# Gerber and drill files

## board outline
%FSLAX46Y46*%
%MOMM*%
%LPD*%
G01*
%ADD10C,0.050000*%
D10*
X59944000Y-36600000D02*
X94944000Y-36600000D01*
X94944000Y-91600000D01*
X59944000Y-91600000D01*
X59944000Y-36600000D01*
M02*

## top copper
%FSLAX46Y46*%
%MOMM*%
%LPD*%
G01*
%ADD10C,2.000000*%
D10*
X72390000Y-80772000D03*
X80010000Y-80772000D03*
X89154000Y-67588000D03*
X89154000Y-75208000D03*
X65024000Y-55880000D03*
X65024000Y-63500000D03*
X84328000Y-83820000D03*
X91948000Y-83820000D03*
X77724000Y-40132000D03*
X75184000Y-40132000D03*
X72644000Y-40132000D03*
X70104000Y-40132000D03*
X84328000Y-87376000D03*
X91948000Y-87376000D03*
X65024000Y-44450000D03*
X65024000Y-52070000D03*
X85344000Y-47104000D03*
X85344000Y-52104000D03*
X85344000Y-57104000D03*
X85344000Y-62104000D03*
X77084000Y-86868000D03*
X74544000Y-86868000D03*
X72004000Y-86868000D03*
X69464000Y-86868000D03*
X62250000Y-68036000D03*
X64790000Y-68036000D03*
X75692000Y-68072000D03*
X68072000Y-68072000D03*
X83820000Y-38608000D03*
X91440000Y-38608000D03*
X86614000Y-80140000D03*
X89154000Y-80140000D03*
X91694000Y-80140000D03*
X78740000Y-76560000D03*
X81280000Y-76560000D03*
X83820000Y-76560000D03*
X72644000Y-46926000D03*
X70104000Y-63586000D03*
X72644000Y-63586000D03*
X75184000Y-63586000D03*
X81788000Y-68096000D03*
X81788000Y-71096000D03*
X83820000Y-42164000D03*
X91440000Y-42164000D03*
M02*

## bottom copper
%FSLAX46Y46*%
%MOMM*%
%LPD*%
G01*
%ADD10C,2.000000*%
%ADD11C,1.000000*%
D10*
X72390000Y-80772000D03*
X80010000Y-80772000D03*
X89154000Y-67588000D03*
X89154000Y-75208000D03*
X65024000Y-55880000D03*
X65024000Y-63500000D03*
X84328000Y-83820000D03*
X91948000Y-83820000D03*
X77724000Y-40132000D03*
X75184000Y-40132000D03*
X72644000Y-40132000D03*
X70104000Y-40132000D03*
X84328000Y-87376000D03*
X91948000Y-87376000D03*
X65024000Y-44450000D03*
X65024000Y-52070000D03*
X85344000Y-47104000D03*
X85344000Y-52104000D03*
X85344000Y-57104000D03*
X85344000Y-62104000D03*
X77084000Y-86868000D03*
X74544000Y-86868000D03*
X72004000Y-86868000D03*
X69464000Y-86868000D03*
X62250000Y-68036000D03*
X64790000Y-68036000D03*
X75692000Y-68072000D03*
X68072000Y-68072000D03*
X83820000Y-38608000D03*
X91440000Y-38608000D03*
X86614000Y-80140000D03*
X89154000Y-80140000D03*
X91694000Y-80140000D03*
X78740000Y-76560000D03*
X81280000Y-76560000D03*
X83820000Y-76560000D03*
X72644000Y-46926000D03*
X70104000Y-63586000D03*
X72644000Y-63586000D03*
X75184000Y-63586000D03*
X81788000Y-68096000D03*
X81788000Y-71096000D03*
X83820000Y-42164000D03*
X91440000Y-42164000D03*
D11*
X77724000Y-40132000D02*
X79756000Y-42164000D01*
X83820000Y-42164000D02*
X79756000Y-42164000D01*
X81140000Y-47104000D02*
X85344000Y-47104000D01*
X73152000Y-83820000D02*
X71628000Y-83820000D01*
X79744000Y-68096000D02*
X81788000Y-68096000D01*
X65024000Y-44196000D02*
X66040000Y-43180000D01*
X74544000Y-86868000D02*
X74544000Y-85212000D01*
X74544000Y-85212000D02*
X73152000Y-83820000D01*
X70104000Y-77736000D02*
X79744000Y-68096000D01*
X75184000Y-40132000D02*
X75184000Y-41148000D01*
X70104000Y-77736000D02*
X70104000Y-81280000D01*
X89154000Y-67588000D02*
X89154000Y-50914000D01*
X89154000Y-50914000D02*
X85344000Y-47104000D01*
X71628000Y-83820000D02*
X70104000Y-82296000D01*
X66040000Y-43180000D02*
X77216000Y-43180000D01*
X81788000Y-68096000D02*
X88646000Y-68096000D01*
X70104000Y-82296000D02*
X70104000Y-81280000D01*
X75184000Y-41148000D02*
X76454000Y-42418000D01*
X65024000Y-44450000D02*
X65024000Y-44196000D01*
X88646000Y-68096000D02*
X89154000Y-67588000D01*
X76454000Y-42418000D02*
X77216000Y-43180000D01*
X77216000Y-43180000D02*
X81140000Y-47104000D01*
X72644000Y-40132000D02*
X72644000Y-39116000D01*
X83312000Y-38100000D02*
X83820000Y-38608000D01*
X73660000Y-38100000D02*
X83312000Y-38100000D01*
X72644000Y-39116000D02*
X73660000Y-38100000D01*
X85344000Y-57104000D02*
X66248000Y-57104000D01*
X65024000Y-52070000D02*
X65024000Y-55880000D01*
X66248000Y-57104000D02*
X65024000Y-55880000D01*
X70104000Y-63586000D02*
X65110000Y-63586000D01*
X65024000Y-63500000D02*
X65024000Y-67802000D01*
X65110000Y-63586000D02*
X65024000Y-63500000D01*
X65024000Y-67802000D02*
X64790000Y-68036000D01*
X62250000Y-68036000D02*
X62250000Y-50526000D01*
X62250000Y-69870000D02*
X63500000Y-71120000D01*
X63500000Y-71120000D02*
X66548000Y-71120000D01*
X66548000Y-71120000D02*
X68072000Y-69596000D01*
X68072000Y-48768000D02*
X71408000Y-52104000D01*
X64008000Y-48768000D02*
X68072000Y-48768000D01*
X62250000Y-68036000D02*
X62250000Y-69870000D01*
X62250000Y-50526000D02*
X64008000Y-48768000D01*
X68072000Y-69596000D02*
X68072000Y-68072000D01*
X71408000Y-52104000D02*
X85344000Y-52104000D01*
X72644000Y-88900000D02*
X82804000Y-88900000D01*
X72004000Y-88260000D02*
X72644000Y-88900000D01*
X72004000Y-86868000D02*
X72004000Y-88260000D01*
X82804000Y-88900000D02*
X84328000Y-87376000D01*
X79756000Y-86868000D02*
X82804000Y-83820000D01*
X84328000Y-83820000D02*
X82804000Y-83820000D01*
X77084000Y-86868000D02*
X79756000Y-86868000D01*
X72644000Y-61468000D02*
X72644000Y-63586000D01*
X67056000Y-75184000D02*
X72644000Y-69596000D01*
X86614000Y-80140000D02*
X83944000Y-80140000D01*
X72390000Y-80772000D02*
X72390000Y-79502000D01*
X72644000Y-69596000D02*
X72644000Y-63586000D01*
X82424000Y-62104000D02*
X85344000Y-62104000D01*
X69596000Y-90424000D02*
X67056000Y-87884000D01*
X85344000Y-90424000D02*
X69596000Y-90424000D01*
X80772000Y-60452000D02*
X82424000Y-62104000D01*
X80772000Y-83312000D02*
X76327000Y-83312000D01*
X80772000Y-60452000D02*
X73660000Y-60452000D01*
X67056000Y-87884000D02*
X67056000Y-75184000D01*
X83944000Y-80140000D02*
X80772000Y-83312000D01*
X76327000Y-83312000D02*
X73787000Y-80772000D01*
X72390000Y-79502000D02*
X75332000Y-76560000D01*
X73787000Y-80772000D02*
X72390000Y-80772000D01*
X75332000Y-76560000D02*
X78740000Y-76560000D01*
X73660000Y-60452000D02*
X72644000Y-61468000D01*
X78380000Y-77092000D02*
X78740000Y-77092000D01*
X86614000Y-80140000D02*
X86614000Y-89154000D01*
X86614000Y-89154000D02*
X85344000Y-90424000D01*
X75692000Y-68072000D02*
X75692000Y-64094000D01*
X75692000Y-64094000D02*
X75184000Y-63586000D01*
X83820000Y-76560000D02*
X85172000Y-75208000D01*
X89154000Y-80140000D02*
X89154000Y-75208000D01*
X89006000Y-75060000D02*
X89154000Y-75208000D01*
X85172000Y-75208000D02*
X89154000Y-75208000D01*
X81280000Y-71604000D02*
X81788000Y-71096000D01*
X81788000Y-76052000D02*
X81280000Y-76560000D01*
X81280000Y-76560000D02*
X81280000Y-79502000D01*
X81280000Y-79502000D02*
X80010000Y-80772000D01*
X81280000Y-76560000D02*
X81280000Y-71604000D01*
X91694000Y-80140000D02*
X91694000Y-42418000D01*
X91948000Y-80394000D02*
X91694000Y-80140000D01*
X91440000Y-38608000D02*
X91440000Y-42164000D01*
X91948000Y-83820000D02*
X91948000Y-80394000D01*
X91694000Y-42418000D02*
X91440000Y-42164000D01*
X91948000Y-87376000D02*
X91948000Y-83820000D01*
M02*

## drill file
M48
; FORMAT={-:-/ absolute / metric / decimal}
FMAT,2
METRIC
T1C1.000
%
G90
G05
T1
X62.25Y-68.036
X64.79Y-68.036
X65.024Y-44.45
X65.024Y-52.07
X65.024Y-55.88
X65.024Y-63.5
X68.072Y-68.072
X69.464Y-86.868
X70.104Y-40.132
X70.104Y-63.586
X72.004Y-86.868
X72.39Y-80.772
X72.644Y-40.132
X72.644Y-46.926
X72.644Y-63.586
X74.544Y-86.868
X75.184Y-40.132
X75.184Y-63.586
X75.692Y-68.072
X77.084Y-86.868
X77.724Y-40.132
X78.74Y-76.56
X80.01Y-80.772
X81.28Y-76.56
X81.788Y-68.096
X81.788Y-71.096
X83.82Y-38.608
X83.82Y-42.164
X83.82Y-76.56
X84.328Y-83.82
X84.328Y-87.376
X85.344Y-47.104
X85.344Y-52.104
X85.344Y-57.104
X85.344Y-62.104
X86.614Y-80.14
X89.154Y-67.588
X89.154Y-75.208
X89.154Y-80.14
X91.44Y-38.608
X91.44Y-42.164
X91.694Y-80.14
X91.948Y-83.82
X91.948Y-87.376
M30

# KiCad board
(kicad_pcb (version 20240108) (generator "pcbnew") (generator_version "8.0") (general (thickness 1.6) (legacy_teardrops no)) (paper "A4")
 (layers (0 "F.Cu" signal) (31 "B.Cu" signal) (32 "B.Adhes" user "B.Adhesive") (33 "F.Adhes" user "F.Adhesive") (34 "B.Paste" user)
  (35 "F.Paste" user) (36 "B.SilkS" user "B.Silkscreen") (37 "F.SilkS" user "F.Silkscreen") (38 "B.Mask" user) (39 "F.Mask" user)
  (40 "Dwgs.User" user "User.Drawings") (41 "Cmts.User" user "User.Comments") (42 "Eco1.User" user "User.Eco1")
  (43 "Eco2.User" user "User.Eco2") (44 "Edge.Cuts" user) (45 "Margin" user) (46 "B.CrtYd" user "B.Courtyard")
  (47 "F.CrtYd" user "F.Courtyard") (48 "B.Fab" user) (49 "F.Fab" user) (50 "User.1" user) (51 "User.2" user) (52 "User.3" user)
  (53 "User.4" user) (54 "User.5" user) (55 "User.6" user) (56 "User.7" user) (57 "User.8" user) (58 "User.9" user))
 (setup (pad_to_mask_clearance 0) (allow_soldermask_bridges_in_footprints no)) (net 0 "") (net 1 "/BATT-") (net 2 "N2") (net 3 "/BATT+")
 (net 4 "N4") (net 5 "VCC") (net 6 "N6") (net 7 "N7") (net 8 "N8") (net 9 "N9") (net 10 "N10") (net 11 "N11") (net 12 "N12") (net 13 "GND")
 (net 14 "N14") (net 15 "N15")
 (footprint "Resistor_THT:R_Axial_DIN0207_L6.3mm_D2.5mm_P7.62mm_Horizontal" (layer "F.Cu") (at 72.39 80.772)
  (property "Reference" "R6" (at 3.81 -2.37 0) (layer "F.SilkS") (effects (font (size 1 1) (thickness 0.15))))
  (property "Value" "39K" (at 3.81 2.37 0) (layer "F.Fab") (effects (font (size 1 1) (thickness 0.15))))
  (pad "1" thru_hole circle (at 0 0) (size 2 2) (drill 1) (layers "*.Cu" "*.Mask") (remove_unused_layers no) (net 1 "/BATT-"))
  (pad "2" thru_hole circle (at 7.62 0) (size 2 2) (drill 1) (layers "*.Cu" "*.Mask") (remove_unused_layers no) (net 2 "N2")))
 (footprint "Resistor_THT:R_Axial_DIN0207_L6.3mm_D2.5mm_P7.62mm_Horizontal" (layer "F.Cu") (at 89.154 67.588 -90)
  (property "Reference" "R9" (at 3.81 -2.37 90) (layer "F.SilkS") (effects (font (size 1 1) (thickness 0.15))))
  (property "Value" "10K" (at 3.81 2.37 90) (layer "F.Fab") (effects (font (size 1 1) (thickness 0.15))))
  (pad "1" thru_hole circle (at 0 0 270) (size 2 2) (drill 1) (layers "*.Cu" "*.Mask") (remove_unused_layers no) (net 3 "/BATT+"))
  (pad "2" thru_hole circle (at 7.62 0 270) (size 2 2) (drill 1) (layers "*.Cu" "*.Mask") (remove_unused_layers no) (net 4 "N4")))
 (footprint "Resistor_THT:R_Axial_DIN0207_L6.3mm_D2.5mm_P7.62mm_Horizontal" (layer "F.Cu") (at 65.024 55.88 -90)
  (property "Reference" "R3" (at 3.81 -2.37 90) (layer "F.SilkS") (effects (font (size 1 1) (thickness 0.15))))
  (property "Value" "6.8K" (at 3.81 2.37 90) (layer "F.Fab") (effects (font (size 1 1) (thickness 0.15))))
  (pad "1" thru_hole circle (at 0 0 270) (size 2 2) (drill 1) (layers "*.Cu" "*.Mask") (remove_unused_layers no) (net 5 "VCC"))
  (pad "2" thru_hole circle (at 7.62 0 270) (size 2 2) (drill 1) (layers "*.Cu" "*.Mask") (remove_unused_layers no) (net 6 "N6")))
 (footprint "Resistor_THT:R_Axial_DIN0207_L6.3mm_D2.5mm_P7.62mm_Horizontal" (layer "F.Cu") (at 84.328 83.82)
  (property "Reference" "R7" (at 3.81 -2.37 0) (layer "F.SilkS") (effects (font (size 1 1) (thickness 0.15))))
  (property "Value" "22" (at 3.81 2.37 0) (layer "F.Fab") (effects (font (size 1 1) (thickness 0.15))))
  (pad "1" thru_hole circle (at 0 0) (size 2 2) (drill 1) (layers "*.Cu" "*.Mask") (remove_unused_layers no) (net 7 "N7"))
  (pad "2" thru_hole circle (at 7.62 0) (size 2 2) (drill 1) (layers "*.Cu" "*.Mask") (remove_unused_layers no) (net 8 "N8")))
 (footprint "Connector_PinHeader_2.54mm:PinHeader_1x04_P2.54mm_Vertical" (layer "F.Cu") (at 77.724 40.132 -90)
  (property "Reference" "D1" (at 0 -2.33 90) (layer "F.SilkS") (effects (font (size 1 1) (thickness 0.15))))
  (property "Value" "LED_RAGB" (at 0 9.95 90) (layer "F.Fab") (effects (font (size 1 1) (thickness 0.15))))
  (pad "1" thru_hole circle (at 0 0 270) (size 2 2) (drill 1) (layers "*.Cu" "*.Mask") (remove_unused_layers no) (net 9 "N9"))
  (pad "2" thru_hole circle (at 0 2.54 270) (size 2 2) (drill 1) (layers "*.Cu" "*.Mask") (remove_unused_layers no) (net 3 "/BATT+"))
  (pad "3" thru_hole circle (at 0 5.08 270) (size 2 2) (drill 1) (layers "*.Cu" "*.Mask") (remove_unused_layers no) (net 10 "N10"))
  (pad "4" thru_hole circle (at 0 7.62 270) (size 2 2) (drill 1) (layers "*.Cu" "*.Mask") (remove_unused_layers no) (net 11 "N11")))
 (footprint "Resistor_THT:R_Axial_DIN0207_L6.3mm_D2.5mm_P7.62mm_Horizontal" (layer "F.Cu") (at 84.328 87.376)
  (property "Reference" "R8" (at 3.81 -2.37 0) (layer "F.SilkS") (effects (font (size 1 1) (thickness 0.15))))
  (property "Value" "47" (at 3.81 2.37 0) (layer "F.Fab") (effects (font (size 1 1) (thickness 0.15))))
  (pad "1" thru_hole circle (at 0 0) (size 2 2) (drill 1) (layers "*.Cu" "*.Mask") (remove_unused_layers no) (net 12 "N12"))
  (pad "2" thru_hole circle (at 7.62 0) (size 2 2) (drill 1) (layers "*.Cu" "*.Mask") (remove_unused_layers no) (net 8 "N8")))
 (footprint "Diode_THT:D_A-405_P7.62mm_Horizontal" (layer "F.Cu") (at 65.024 44.45 -90)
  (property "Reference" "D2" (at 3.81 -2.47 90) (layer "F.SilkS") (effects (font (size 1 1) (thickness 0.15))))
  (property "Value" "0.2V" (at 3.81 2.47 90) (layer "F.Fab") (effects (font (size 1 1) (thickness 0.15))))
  (pad "1" thru_hole circle (at 0 0 270) (size 2 2) (drill 1) (layers "*.Cu" "*.Mask") (remove_unused_layers no) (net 3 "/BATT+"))
  (pad "2" thru_hole circle (at 7.62 0 270) (size 2 2) (drill 1) (layers "*.Cu" "*.Mask") (remove_unused_layers no) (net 5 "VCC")))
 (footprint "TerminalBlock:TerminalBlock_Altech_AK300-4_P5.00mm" (layer "F.Cu") (at 85.344 47.104 -90)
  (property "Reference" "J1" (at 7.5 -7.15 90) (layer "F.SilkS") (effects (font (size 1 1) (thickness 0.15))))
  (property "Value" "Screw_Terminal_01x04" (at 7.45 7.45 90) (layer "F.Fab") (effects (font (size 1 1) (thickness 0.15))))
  (pad "1" thru_hole circle (at 0 0 270) (size 2 2) (drill 1) (layers "*.Cu" "*.Mask") (remove_unused_layers no) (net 3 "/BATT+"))
  (pad "2" thru_hole circle (at 5 0 270) (size 2 2) (drill 1) (layers "*.Cu" "*.Mask") (remove_unused_layers no) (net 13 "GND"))
  (pad "3" thru_hole circle (at 10 0 270) (size 2 2) (drill 1) (layers "*.Cu" "*.Mask") (remove_unused_layers no) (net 5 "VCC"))
  (pad "4" thru_hole circle (at 15 0 270) (size 2 2) (drill 1) (layers "*.Cu" "*.Mask") (remove_unused_layers no) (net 1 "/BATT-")))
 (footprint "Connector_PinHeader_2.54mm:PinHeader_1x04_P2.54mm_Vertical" (layer "F.Cu") (at 77.084 86.868 -90)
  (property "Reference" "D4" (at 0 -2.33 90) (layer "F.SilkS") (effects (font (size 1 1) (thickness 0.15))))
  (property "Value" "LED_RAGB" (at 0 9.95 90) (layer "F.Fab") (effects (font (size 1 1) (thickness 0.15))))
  (pad "1" thru_hole circle (at 0 0 270) (size 2 2) (drill 1) (layers "*.Cu" "*.Mask") (remove_unused_layers no) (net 7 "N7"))
  (pad "2" thru_hole circle (at 0 2.54 270) (size 2 2) (drill 1) (layers "*.Cu" "*.Mask") (remove_unused_layers no) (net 3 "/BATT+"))
  (pad "3" thru_hole circle (at 0 5.08 270) (size 2 2) (drill 1) (layers "*.Cu" "*.Mask") (remove_unused_layers no) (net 12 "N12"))
  (pad "4" thru_hole circle (at 0 7.62 270) (size 2 2) (drill 1) (layers "*.Cu" "*.Mask") (remove_unused_layers no) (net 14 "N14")))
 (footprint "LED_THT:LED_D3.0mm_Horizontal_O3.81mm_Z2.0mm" (layer "F.Cu") (at 62.25 68.036)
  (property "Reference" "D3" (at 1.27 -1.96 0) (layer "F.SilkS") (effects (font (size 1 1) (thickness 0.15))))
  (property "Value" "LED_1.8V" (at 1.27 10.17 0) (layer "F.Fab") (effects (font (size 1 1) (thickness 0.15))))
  (pad "1" thru_hole circle (at 0 0) (size 2 2) (drill 1) (layers "*.Cu" "*.Mask") (remove_unused_layers no) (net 13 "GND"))
  (pad "2" thru_hole circle (at 2.54 0) (size 2 2) (drill 1) (layers "*.Cu" "*.Mask") (remove_unused_layers no) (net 6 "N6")))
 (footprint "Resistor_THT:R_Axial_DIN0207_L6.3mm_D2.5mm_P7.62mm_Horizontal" (layer "F.Cu") (at 75.692 68.072 180)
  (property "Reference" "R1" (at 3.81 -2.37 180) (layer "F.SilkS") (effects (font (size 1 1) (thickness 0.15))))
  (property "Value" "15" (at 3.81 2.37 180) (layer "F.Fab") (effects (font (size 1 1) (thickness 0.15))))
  (pad "1" thru_hole circle (at 0 0 180) (size 2 2) (drill 1) (layers "*.Cu" "*.Mask") (remove_unused_layers no) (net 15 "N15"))
  (pad "2" thru_hole circle (at 7.62 0 180) (size 2 2) (drill 1) (layers "*.Cu" "*.Mask") (remove_unused_layers no) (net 13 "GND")))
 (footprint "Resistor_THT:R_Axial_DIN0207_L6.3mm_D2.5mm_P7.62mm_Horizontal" (layer "F.Cu") (at 83.82 38.608)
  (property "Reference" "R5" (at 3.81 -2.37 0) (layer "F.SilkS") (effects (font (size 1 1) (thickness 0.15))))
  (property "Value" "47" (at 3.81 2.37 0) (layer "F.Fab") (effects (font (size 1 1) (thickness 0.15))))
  (pad "1" thru_hole circle (at 0 0) (size 2 2) (drill 1) (layers "*.Cu" "*.Mask") (remove_unused_layers no) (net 10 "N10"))
  (pad "2" thru_hole circle (at 7.62 0) (size 2 2) (drill 1) (layers "*.Cu" "*.Mask") (remove_unused_layers no) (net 8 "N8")))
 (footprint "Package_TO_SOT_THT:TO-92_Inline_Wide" (layer "F.Cu") (at 86.614 80.14)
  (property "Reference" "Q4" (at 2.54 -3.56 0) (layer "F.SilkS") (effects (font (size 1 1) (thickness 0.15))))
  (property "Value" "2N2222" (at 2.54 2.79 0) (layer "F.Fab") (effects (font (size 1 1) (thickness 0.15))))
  (pad "1" thru_hole circle (at 0 0) (size 2 2) (drill 1) (layers "*.Cu" "*.Mask") (remove_unused_layers no) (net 1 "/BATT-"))
  (pad "2" thru_hole circle (at 2.54 0) (size 2 2) (drill 1) (layers "*.Cu" "*.Mask") (remove_unused_layers no) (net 4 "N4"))
  (pad "3" thru_hole circle (at 5.08 0) (size 2 2) (drill 1) (layers "*.Cu" "*.Mask") (remove_unused_layers no) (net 8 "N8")))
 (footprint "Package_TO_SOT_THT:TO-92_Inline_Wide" (layer "F.Cu") (at 78.74 76.56)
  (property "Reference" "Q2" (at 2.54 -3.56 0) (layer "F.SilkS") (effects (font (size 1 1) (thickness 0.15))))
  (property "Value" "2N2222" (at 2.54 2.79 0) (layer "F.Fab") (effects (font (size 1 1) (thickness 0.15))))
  (pad "1" thru_hole circle (at 0 0) (size 2 2) (drill 1) (layers "*.Cu" "*.Mask") (remove_unused_layers no) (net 1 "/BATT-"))
  (pad "2" thru_hole circle (at 2.54 0) (size 2 2) (drill 1) (layers "*.Cu" "*.Mask") (remove_unused_layers no) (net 2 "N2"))
  (pad "3" thru_hole circle (at 5.08 0) (size 2 2) (drill 1) (layers "*.Cu" "*.Mask") (remove_unused_layers no) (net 4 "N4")))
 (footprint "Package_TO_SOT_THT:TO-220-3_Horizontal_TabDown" (layer "F.Cu") (at 70.104 63.586)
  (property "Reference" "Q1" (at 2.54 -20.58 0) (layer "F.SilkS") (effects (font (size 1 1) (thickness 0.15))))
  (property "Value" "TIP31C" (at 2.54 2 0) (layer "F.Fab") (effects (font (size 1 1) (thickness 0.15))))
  (pad "" thru_hole circle (at 2.54 -16.66) (size 2 2) (drill 1) (layers "*.Cu" "*.Mask") (remove_unused_layers no))
  (pad "1" thru_hole circle (at 0 0) (size 2 2) (drill 1) (layers "*.Cu" "*.Mask") (remove_unused_layers no) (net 6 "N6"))
  (pad "2" thru_hole circle (at 2.54 0) (size 2 2) (drill 1) (layers "*.Cu" "*.Mask") (remove_unused_layers no) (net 1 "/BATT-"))
  (pad "3" thru_hole circle (at 5.08 0) (size 2 2) (drill 1) (layers "*.Cu" "*.Mask") (remove_unused_layers no) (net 15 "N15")))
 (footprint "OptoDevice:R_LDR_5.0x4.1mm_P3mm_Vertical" (layer "F.Cu") (at 81.788 68.096 -90)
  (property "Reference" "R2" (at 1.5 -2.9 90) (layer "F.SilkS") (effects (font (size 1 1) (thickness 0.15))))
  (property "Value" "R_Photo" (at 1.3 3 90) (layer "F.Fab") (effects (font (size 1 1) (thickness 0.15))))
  (pad "1" thru_hole circle (at 0 0 270) (size 2 2) (drill 1) (layers "*.Cu" "*.Mask") (remove_unused_layers no) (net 3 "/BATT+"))
  (pad "2" thru_hole circle (at 3 0 270) (size 2 2) (drill 1) (layers "*.Cu" "*.Mask") (remove_unused_layers no) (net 2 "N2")))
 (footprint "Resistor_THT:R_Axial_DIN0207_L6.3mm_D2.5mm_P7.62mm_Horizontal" (layer "F.Cu") (at 83.82 42.164)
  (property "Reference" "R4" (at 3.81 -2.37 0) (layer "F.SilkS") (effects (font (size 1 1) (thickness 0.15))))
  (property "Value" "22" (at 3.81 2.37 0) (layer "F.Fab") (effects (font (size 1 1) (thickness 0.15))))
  (pad "1" thru_hole circle (at 0 0) (size 2 2) (drill 1) (layers "*.Cu" "*.Mask") (remove_unused_layers no) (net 9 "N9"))
  (pad "2" thru_hole circle (at 7.62 0) (size 2 2) (drill 1) (layers "*.Cu" "*.Mask") (remove_unused_layers no) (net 8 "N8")))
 (gr_rect (start 59.944 36.6) (end 94.944 91.6) (stroke (width 0.05) (type default)) (fill none) (layer "Edge.Cuts"))
 (segment (start 77.724 40.132) (end 79.756 42.164) (width 1) (layer "B.Cu") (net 9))
 (segment (start 83.82 42.164) (end 79.756 42.164) (width 1) (layer "B.Cu") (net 9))
 (segment (start 81.14 47.104) (end 85.344 47.104) (width 1) (layer "B.Cu") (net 3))
 (segment (start 73.152 83.82) (end 71.628 83.82) (width 1) (layer "B.Cu") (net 3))
 (segment (start 79.744 68.096) (end 81.788 68.096) (width 1) (layer "B.Cu") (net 3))
 (segment (start 65.024 44.196) (end 66.04 43.18) (width 1) (layer "B.Cu") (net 3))
 (segment (start 74.544 86.868) (end 74.544 85.212) (width 1) (layer "B.Cu") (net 3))
 (segment (start 74.544 85.212) (end 73.152 83.82) (width 1) (layer "B.Cu") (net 3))
 (segment (start 70.104 77.736) (end 79.744 68.096) (width 1) (layer "B.Cu") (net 3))
 (segment (start 75.184 40.132) (end 75.184 41.148) (width 1) (layer "B.Cu") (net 3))
 (segment (start 70.104 77.736) (end 70.104 81.28) (width 1) (layer "B.Cu") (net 3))
 (segment (start 89.154 67.588) (end 89.154 50.914) (width 1) (layer "B.Cu") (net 3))
 (segment (start 89.154 50.914) (end 85.344 47.104) (width 1) (layer "B.Cu") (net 3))
 (segment (start 71.628 83.82) (end 70.104 82.296) (width 1) (layer "B.Cu") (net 3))
 (segment (start 66.04 43.18) (end 77.216 43.18) (width 1) (layer "B.Cu") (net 3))
 (segment (start 81.788 68.096) (end 88.646 68.096) (width 1) (layer "B.Cu") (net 3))
 (segment (start 70.104 82.296) (end 70.104 81.28) (width 1) (layer "B.Cu") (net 3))
 (segment (start 75.184 41.148) (end 76.454 42.418) (width 1) (layer "B.Cu") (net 3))
 (segment (start 65.024 44.45) (end 65.024 44.196) (width 1) (layer "B.Cu") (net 3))
 (segment (start 88.646 68.096) (end 89.154 67.588) (width 1) (layer "B.Cu") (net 3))
 (segment (start 76.454 42.418) (end 77.216 43.18) (width 1) (layer "B.Cu") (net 3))
 (segment (start 77.216 43.18) (end 81.14 47.104) (width 1) (layer "B.Cu") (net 3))
 (segment (start 72.644 40.132) (end 72.644 39.116) (width 1) (layer "B.Cu") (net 10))
 (segment (start 83.312 38.1) (end 83.82 38.608) (width 1) (layer "B.Cu") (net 10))
 (segment (start 73.66 38.1) (end 83.312 38.1) (width 1) (layer "B.Cu") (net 10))
 (segment (start 72.644 39.116) (end 73.66 38.1) (width 1) (layer "B.Cu") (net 10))
 (segment (start 85.344 57.104) (end 66.248 57.104) (width 1) (layer "B.Cu") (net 5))
 (segment (start 65.024 52.07) (end 65.024 55.88) (width 1) (layer "B.Cu") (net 5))
 (segment (start 66.248 57.104) (end 65.024 55.88) (width 1) (layer "B.Cu") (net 5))
 (segment (start 70.104 63.586) (end 65.11 63.586) (width 1) (layer "B.Cu") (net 6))
 (segment (start 65.024 63.5) (end 65.024 67.802) (width 1) (layer "B.Cu") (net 6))
 (segment (start 65.11 63.586) (end 65.024 63.5) (width 1) (layer "B.Cu") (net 6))
 (segment (start 65.024 67.802) (end 64.79 68.036) (width 1) (layer "B.Cu") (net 6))
 (segment (start 62.25 68.036) (end 62.25 50.526) (width 1) (layer "B.Cu") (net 13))
 (segment (start 62.25 69.87) (end 63.5 71.12) (width 1) (layer "B.Cu") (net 13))
 (segment (start 63.5 71.12) (end 66.548 71.12) (width 1) (layer "B.Cu") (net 13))
 (segment (start 66.548 71.12) (end 68.072 69.596) (width 1) (layer "B.Cu") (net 13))
 (segment (start 68.072 48.768) (end 71.408 52.104) (width 1) (layer "B.Cu") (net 13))
 (segment (start 64.008 48.768) (end 68.072 48.768) (width 1) (layer "B.Cu") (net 13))
 (segment (start 62.25 68.036) (end 62.25 69.87) (width 1) (layer "B.Cu") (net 13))
 (segment (start 62.25 50.526) (end 64.008 48.768) (width 1) (layer "B.Cu") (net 13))
 (segment (start 68.072 69.596) (end 68.072 68.072) (width 1) (layer "B.Cu") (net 13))
 (segment (start 71.408 52.104) (end 85.344 52.104) (width 1) (layer "B.Cu") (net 13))
 (segment (start 72.644 88.9) (end 82.804 88.9) (width 1) (layer "B.Cu") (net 12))
 (segment (start 72.004 88.26) (end 72.644 88.9) (width 1) (layer "B.Cu") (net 12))
 (segment (start 72.004 86.868) (end 72.004 88.26) (width 1) (layer "B.Cu") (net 12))
 (segment (start 82.804 88.9) (end 84.328 87.376) (width 1) (layer "B.Cu") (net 12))
 (segment (start 79.756 86.868) (end 82.804 83.82) (width 1) (layer "B.Cu") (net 7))
 (segment (start 84.328 83.82) (end 82.804 83.82) (width 1) (layer "B.Cu") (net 7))
 (segment (start 77.084 86.868) (end 79.756 86.868) (width 1) (layer "B.Cu") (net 7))
 (segment (start 72.644 61.468) (end 72.644 63.586) (width 1) (layer "B.Cu") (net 1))
 (segment (start 67.056 75.184) (end 72.644 69.596) (width 1) (layer "B.Cu") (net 1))
 (segment (start 86.614 80.14) (end 83.944 80.14) (width 1) (layer "B.Cu") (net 1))
 (segment (start 72.39 80.772) (end 72.39 79.502) (width 1) (layer "B.Cu") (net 1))
 (segment (start 72.644 69.596) (end 72.644 63.586) (width 1) (layer "B.Cu") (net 1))
 (segment (start 82.424 62.104) (end 85.344 62.104) (width 1) (layer "B.Cu") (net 1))
 (segment (start 69.596 90.424) (end 67.056 87.884) (width 1) (layer "B.Cu") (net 1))
 (segment (start 85.344 90.424) (end 69.596 90.424) (width 1) (layer "B.Cu") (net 1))
 (segment (start 80.772 60.452) (end 82.424 62.104) (width 1) (layer "B.Cu") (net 1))
 (segment (start 80.772 83.312) (end 76.327 83.312) (width 1) (layer "B.Cu") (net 1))
 (segment (start 80.772 60.452) (end 73.66 60.452) (width 1) (layer "B.Cu") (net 1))
 (segment (start 67.056 87.884) (end 67.056 75.184) (width 1) (layer "B.Cu") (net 1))
 (segment (start 83.944 80.14) (end 80.772 83.312) (width 1) (layer "B.Cu") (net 1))
 (segment (start 76.327 83.312) (end 73.787 80.772) (width 1) (layer "B.Cu") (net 1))
 (segment (start 72.39 79.502) (end 75.332 76.56) (width 1) (layer "B.Cu") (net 1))
 (segment (start 73.787 80.772) (end 72.39 80.772) (width 1) (layer "B.Cu") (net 1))
 (segment (start 75.332 76.56) (end 78.74 76.56) (width 1) (layer "B.Cu") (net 1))
 (segment (start 73.66 60.452) (end 72.644 61.468) (width 1) (layer "B.Cu") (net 1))
 (segment (start 78.38 77.092) (end 78.74 77.092) (width 1) (layer "B.Cu") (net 1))
 (segment (start 86.614 80.14) (end 86.614 89.154) (width 1) (layer "B.Cu") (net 1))
 (segment (start 86.614 89.154) (end 85.344 90.424) (width 1) (layer "B.Cu") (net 1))
 (segment (start 75.692 68.072) (end 75.692 64.094) (width 1) (layer "B.Cu") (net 15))
 (segment (start 75.692 64.094) (end 75.184 63.586) (width 1) (layer "B.Cu") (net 15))
 (segment (start 83.82 76.56) (end 85.172 75.208) (width 1) (layer "B.Cu") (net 4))
 (segment (start 89.154 80.14) (end 89.154 75.208) (width 1) (layer "B.Cu") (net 4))
 (segment (start 89.006 75.06) (end 89.154 75.208) (width 1) (layer "B.Cu") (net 4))
 (segment (start 85.172 75.208) (end 89.154 75.208) (width 1) (layer "B.Cu") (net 4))
 (segment (start 81.28 71.604) (end 81.788 71.096) (width 1) (layer "B.Cu") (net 2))
 (segment (start 81.788 76.052) (end 81.28 76.56) (width 1) (layer "B.Cu") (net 2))
 (segment (start 81.28 76.56) (end 81.28 79.502) (width 1) (layer "B.Cu") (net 2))
 (segment (start 81.28 79.502) (end 80.01 80.772) (width 1) (layer "B.Cu") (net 2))
 (segment (start 81.28 76.56) (end 81.28 71.604) (width 1) (layer "B.Cu") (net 2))
 (segment (start 91.694 80.14) (end 91.694 42.418) (width 1) (layer "B.Cu") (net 8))
 (segment (start 91.948 80.394) (end 91.694 80.14) (width 1) (layer "B.Cu") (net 8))
 (segment (start 91.44 38.608) (end 91.44 42.164) (width 1) (layer "B.Cu") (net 8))
 (segment (start 91.948 83.82) (end 91.948 80.394) (width 1) (layer "B.Cu") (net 8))
 (segment (start 91.694 42.418) (end 91.44 42.164) (width 1) (layer "B.Cu") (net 8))
 (segment (start 91.948 87.376) (end 91.948 83.82) (width 1) (layer "B.Cu") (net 8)))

